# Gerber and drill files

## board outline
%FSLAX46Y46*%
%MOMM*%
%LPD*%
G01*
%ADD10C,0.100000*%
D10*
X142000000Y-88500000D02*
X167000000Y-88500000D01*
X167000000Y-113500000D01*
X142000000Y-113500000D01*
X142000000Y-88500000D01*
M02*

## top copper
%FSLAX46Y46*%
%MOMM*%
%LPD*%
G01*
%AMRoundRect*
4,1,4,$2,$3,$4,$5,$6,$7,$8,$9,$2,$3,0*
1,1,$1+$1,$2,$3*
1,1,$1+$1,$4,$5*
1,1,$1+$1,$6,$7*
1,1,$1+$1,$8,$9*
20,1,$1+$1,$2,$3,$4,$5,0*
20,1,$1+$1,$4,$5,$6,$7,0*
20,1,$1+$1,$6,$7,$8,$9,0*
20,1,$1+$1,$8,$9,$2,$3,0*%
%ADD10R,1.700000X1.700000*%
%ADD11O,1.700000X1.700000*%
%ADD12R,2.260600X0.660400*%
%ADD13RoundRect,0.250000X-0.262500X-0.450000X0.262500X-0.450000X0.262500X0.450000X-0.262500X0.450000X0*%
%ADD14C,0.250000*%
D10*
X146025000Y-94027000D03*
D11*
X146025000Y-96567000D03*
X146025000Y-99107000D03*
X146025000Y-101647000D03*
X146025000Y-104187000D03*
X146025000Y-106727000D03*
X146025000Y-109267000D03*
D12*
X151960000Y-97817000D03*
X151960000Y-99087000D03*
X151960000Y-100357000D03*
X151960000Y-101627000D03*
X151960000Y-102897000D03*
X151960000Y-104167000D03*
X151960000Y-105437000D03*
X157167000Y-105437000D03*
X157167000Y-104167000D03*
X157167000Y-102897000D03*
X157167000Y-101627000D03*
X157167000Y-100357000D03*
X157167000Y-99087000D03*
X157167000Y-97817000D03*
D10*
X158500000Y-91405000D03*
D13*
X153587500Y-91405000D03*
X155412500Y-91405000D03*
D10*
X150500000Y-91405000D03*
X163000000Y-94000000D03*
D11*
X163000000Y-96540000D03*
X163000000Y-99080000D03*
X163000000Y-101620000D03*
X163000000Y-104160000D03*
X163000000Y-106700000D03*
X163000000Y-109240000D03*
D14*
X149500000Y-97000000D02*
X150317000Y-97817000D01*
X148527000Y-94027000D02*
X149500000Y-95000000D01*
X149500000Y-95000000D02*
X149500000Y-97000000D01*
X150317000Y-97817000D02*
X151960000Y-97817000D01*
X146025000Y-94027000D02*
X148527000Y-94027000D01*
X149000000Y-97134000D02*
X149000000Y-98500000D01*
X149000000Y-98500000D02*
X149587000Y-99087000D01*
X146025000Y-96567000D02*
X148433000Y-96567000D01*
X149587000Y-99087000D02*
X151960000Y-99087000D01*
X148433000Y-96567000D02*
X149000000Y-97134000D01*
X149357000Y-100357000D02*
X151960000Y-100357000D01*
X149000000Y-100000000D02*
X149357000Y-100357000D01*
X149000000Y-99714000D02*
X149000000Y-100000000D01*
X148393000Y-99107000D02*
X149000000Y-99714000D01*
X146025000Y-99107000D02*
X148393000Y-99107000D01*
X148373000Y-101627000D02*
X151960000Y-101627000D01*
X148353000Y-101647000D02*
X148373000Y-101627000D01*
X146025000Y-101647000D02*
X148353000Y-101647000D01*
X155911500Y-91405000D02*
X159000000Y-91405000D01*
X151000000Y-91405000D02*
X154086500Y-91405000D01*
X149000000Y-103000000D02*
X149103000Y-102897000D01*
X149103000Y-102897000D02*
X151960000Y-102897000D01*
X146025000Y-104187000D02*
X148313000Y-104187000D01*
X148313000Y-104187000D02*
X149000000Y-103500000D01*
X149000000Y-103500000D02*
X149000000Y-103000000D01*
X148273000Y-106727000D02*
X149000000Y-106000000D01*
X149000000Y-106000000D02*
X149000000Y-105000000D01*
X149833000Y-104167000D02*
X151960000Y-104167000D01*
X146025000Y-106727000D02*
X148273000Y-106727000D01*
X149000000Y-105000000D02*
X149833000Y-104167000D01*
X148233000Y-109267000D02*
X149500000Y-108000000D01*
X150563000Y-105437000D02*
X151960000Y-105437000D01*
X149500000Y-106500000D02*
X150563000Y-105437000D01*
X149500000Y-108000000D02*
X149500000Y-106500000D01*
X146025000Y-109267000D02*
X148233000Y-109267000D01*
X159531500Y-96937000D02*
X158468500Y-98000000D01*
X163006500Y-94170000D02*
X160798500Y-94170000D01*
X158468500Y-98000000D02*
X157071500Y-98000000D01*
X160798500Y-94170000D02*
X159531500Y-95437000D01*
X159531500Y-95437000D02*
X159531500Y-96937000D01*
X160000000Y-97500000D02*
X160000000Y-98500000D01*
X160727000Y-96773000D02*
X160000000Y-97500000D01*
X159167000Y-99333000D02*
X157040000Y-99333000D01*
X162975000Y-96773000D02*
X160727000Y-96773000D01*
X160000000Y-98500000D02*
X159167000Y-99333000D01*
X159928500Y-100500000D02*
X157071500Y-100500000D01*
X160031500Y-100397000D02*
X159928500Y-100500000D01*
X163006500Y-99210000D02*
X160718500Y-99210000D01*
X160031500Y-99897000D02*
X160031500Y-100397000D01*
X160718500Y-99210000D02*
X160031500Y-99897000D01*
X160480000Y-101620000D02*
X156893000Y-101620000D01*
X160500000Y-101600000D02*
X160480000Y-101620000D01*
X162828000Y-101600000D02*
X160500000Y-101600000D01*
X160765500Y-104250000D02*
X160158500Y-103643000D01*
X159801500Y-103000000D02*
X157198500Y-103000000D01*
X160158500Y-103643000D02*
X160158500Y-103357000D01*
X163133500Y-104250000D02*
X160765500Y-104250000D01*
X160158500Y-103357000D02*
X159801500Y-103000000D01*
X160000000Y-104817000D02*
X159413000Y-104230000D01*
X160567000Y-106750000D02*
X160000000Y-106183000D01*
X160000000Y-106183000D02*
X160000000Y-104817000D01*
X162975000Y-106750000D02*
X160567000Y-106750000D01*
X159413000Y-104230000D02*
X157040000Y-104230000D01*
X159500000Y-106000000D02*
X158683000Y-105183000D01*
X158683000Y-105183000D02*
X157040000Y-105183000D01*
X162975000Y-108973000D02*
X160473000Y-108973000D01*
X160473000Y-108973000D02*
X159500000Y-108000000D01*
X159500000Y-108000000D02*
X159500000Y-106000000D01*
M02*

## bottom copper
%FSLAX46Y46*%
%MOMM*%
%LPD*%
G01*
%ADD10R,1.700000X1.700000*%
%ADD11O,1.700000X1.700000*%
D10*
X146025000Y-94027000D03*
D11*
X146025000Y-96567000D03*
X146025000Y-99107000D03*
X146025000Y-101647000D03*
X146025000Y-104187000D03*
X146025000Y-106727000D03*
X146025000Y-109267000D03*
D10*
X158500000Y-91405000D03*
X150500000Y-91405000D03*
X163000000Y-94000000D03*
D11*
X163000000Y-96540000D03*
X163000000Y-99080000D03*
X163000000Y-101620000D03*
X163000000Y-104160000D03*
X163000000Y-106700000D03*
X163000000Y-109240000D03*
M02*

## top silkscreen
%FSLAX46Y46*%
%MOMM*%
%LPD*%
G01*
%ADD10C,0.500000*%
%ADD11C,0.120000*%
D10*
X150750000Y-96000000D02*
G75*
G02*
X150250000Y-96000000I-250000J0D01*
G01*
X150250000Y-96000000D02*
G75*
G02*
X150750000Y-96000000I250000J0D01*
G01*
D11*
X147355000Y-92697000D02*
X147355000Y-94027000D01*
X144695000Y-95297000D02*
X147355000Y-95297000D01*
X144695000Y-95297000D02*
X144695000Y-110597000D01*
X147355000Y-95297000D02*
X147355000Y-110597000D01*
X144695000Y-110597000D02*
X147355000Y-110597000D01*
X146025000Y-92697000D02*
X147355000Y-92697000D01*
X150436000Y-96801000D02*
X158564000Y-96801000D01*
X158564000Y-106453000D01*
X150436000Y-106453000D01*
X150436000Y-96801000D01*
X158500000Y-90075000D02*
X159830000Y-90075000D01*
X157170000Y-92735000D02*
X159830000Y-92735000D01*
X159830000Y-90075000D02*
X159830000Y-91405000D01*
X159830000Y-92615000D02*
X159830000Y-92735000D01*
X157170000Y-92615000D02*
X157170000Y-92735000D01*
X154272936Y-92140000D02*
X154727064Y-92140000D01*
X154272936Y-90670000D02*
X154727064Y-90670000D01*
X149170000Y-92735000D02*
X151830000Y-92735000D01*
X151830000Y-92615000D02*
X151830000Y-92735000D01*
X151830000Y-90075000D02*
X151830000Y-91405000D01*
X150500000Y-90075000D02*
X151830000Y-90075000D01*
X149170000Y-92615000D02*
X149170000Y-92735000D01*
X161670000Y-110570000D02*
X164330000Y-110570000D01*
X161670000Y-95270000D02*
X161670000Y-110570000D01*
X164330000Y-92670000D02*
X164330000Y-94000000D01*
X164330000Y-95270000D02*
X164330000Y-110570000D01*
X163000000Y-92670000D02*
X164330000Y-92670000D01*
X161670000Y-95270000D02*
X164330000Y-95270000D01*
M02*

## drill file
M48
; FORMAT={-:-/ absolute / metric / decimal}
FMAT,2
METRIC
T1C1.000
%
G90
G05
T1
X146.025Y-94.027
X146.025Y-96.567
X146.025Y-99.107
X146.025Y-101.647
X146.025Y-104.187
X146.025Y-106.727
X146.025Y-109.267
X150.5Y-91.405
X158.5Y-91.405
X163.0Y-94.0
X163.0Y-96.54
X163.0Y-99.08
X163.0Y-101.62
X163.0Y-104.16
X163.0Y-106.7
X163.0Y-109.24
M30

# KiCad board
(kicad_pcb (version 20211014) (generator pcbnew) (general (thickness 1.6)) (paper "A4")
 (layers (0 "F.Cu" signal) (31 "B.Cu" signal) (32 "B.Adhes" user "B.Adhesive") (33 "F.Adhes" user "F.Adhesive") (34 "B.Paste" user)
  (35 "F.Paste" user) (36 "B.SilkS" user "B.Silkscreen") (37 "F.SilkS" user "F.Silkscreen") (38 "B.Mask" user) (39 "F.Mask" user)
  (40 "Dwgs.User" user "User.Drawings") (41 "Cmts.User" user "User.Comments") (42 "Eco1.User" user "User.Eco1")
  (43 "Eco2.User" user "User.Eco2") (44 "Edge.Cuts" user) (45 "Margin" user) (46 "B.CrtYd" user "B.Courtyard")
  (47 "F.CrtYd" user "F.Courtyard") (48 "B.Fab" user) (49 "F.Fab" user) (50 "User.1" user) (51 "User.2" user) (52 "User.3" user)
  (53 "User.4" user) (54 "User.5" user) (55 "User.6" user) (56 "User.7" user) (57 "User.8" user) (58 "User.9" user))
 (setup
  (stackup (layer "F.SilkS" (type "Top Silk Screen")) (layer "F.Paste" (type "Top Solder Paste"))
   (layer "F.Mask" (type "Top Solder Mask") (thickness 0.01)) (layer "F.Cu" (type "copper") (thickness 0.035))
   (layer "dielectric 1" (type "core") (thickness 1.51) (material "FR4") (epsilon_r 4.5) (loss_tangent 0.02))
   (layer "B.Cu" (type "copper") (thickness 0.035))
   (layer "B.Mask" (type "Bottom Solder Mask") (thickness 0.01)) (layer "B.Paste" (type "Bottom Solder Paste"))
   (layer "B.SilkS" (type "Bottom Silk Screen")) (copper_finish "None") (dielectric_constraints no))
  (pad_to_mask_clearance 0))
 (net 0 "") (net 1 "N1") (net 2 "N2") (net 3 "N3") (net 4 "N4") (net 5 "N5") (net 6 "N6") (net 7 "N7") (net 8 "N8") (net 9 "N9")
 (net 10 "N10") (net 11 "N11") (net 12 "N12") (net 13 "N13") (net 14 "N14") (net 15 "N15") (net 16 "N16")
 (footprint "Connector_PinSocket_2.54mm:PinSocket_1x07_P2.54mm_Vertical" (layer "F.Cu") (at 146.025 94.027)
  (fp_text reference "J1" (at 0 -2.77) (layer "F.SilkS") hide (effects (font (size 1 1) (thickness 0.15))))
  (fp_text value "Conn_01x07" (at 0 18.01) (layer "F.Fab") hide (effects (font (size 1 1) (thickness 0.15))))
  (fp_line (start 1.33 -1.33) (end 1.33 0) (layer "F.SilkS") (width 0.12))
  (fp_line (start -1.33 1.27) (end 1.33 1.27) (layer "F.SilkS") (width 0.12))
  (fp_line (start -1.33 1.27) (end -1.33 16.57) (layer "F.SilkS") (width 0.12))
  (fp_line (start 1.33 1.27) (end 1.33 16.57) (layer "F.SilkS") (width 0.12))
  (fp_line (start -1.33 16.57) (end 1.33 16.57) (layer "F.SilkS") (width 0.12))
  (fp_line (start 0 -1.33) (end 1.33 -1.33) (layer "F.SilkS") (width 0.12))
  (pad "1" thru_hole rect (at 0 0) (size 1.7 1.7) (drill 1) (layers *.Cu *.Mask) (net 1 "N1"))
  (pad "2" thru_hole oval (at 0 2.54) (size 1.7 1.7) (drill 1) (layers *.Cu *.Mask) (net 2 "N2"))
  (pad "3" thru_hole oval (at 0 5.08) (size 1.7 1.7) (drill 1) (layers *.Cu *.Mask) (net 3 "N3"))
  (pad "4" thru_hole oval (at 0 7.62) (size 1.7 1.7) (drill 1) (layers *.Cu *.Mask) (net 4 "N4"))
  (pad "5" thru_hole oval (at 0 10.16) (size 1.7 1.7) (drill 1) (layers *.Cu *.Mask) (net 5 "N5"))
  (pad "6" thru_hole oval (at 0 12.7) (size 1.7 1.7) (drill 1) (layers *.Cu *.Mask) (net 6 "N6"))
  (pad "7" thru_hole oval (at 0 15.24) (size 1.7 1.7) (drill 1) (layers *.Cu *.Mask) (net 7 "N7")))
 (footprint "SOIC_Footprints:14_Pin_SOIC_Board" (layer "F.Cu") (at 154.627 101.5)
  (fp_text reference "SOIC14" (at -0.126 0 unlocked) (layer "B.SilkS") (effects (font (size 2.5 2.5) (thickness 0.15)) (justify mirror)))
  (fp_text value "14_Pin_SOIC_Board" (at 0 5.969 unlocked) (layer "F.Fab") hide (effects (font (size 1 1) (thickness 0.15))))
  (fp_rect (start -4.191 -4.699) (end 3.937 4.953) (layer "F.SilkS") (width 0.12) (fill none))
  (pad "1" smd rect (at -2.667 -3.683) (size 2.2606 0.6604) (layers "F.Cu" "F.Paste" "F.Mask") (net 1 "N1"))
  (pad "2" smd rect (at -2.667 -2.413) (size 2.2606 0.6604) (layers "F.Cu" "F.Paste" "F.Mask") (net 2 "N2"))
  (pad "3" smd rect (at -2.667 -1.143) (size 2.2606 0.6604) (layers "F.Cu" "F.Paste" "F.Mask") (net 3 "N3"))
  (pad "4" smd rect (at -2.667 0.127) (size 2.2606 0.6604) (layers "F.Cu" "F.Paste" "F.Mask") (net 4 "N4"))
  (pad "5" smd rect (at -2.667 1.397) (size 2.2606 0.6604) (layers "F.Cu" "F.Paste" "F.Mask") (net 5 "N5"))
  (pad "6" smd rect (at -2.667 2.667) (size 2.2606 0.6604) (layers "F.Cu" "F.Paste" "F.Mask") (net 6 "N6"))
  (pad "7" smd rect (at -2.667 3.937) (size 2.2606 0.6604) (layers "F.Cu" "F.Paste" "F.Mask") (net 7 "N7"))
  (pad "8" smd rect (at 2.54 3.937) (size 2.2606 0.6604) (layers "F.Cu" "F.Paste" "F.Mask") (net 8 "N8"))
  (pad "9" smd rect (at 2.54 2.667) (size 2.2606 0.6604) (layers "F.Cu" "F.Paste" "F.Mask") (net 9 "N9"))
  (pad "10" smd rect (at 2.54 1.397) (size 2.2606 0.6604) (layers "F.Cu" "F.Paste" "F.Mask") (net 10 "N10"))
  (pad "11" smd rect (at 2.54 0.127) (size 2.2606 0.6604) (layers "F.Cu" "F.Paste" "F.Mask") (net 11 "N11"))
  (pad "12" smd rect (at 2.54 -1.143) (size 2.2606 0.6604) (layers "F.Cu" "F.Paste" "F.Mask") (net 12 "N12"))
  (pad "13" smd rect (at 2.54 -2.413) (size 2.2606 0.6604) (layers "F.Cu" "F.Paste" "F.Mask") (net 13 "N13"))
  (pad "14" smd rect (at 2.54 -3.683) (size 2.2606 0.6604) (layers "F.Cu" "F.Paste" "F.Mask") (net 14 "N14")))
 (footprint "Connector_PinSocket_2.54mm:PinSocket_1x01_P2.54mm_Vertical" (layer "F.Cu") (at 158.5 91.405)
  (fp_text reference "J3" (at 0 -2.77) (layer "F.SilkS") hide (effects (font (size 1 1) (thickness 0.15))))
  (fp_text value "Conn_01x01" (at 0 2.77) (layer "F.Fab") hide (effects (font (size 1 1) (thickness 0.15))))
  (fp_line (start 0 -1.33) (end 1.33 -1.33) (layer "F.SilkS") (width 0.12))
  (fp_line (start -1.33 1.33) (end 1.33 1.33) (layer "F.SilkS") (width 0.12))
  (fp_line (start 1.33 -1.33) (end 1.33 0) (layer "F.SilkS") (width 0.12))
  (fp_line (start 1.33 1.21) (end 1.33 1.33) (layer "F.SilkS") (width 0.12))
  (fp_line (start -1.33 1.21) (end -1.33 1.33) (layer "F.SilkS") (width 0.12))
  (pad "1" thru_hole rect (at 0 0) (size 1.7 1.7) (drill 1) (layers *.Cu *.Mask) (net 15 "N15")))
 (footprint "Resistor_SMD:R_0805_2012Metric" (layer "F.Cu") (at 154.5 91.405)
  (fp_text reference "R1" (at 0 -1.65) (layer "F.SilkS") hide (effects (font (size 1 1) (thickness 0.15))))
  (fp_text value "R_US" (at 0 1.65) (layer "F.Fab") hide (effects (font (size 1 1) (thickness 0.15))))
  (fp_line (start -0.227064 0.735) (end 0.227064 0.735) (layer "F.SilkS") (width 0.12))
  (fp_line (start -0.227064 -0.735) (end 0.227064 -0.735) (layer "F.SilkS") (width 0.12))
  (pad "1" smd roundrect (at -0.9125 0) (size 1.025 1.4) (layers "F.Cu" "F.Paste" "F.Mask") (roundrect_rratio 0.243902) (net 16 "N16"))
  (pad "2" smd roundrect (at 0.9125 0) (size 1.025 1.4) (layers "F.Cu" "F.Paste" "F.Mask") (roundrect_rratio 0.243902) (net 15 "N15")))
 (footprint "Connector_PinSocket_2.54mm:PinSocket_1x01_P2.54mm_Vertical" (layer "F.Cu") (at 150.5 91.405)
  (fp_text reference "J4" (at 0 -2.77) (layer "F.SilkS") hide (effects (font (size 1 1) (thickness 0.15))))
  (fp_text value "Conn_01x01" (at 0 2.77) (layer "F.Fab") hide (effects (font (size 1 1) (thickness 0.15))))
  (fp_line (start -1.33 1.33) (end 1.33 1.33) (layer "F.SilkS") (width 0.12))
  (fp_line (start 1.33 1.21) (end 1.33 1.33) (layer "F.SilkS") (width 0.12))
  (fp_line (start 1.33 -1.33) (end 1.33 0) (layer "F.SilkS") (width 0.12))
  (fp_line (start 0 -1.33) (end 1.33 -1.33) (layer "F.SilkS") (width 0.12))
  (fp_line (start -1.33 1.21) (end -1.33 1.33) (layer "F.SilkS") (width 0.12))
  (pad "1" thru_hole rect (at 0 0) (size 1.7 1.7) (drill 1) (layers *.Cu *.Mask) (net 16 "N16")))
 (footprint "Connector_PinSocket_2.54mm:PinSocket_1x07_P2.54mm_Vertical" (layer "F.Cu") (at 163 94)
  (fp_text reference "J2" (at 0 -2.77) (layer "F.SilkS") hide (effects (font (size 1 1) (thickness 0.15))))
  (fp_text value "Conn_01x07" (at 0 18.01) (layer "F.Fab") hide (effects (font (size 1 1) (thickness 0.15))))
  (fp_line (start -1.33 16.57) (end 1.33 16.57) (layer "F.SilkS") (width 0.12))
  (fp_line (start -1.33 1.27) (end -1.33 16.57) (layer "F.SilkS") (width 0.12))
  (fp_line (start 1.33 -1.33) (end 1.33 0) (layer "F.SilkS") (width 0.12))
  (fp_line (start 1.33 1.27) (end 1.33 16.57) (layer "F.SilkS") (width 0.12))
  (fp_line (start 0 -1.33) (end 1.33 -1.33) (layer "F.SilkS") (width 0.12))
  (fp_line (start -1.33 1.27) (end 1.33 1.27) (layer "F.SilkS") (width 0.12))
  (pad "1" thru_hole rect (at 0 0) (size 1.7 1.7) (drill 1) (layers *.Cu *.Mask) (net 14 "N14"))
  (pad "2" thru_hole oval (at 0 2.54) (size 1.7 1.7) (drill 1) (layers *.Cu *.Mask) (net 13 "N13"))
  (pad "3" thru_hole oval (at 0 5.08) (size 1.7 1.7) (drill 1) (layers *.Cu *.Mask) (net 12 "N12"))
  (pad "4" thru_hole oval (at 0 7.62) (size 1.7 1.7) (drill 1) (layers *.Cu *.Mask) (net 11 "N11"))
  (pad "5" thru_hole oval (at 0 10.16) (size 1.7 1.7) (drill 1) (layers *.Cu *.Mask) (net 10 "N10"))
  (pad "6" thru_hole oval (at 0 12.7) (size 1.7 1.7) (drill 1) (layers *.Cu *.Mask) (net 9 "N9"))
  (pad "7" thru_hole oval (at 0 15.24) (size 1.7 1.7) (drill 1) (layers *.Cu *.Mask) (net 8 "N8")))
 (gr_circle (center 150.5 96) (end 150.9 96) (layer "F.SilkS") (width 0.2) (fill solid))
 (gr_rect (start 142 88.5) (end 167 113.5) (layer "Edge.Cuts") (width 0.1) (fill none))
 (segment (start 149.5 97) (end 150.317 97.817) (width 0.25) (layer "F.Cu") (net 1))
 (segment (start 148.527 94.027) (end 149.5 95) (width 0.25) (layer "F.Cu") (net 1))
 (segment (start 149.5 95) (end 149.5 97) (width 0.25) (layer "F.Cu") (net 1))
 (segment (start 150.317 97.817) (end 151.96 97.817) (width 0.25) (layer "F.Cu") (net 1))
 (segment (start 146.025 94.027) (end 148.527 94.027) (width 0.25) (layer "F.Cu") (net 1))
 (segment (start 149 97.134) (end 149 98.5) (width 0.25) (layer "F.Cu") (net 2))
 (segment (start 149 98.5) (end 149.587 99.087) (width 0.25) (layer "F.Cu") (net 2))
 (segment (start 146.025 96.567) (end 148.433 96.567) (width 0.25) (layer "F.Cu") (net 2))
 (segment (start 149.587 99.087) (end 151.96 99.087) (width 0.25) (layer "F.Cu") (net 2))
 (segment (start 148.433 96.567) (end 149 97.134) (width 0.25) (layer "F.Cu") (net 2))
 (segment (start 149.357 100.357) (end 151.96 100.357) (width 0.25) (layer "F.Cu") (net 3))
 (segment (start 149 100) (end 149.357 100.357) (width 0.25) (layer "F.Cu") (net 3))
 (segment (start 149 99.714) (end 149 100) (width 0.25) (layer "F.Cu") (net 3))
 (segment (start 148.393 99.107) (end 149 99.714) (width 0.25) (layer "F.Cu") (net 3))
 (segment (start 146.025 99.107) (end 148.393 99.107) (width 0.25) (layer "F.Cu") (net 3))
 (segment (start 148.373 101.627) (end 151.96 101.627) (width 0.25) (layer "F.Cu") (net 4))
 (segment (start 148.353 101.647) (end 148.373 101.627) (width 0.25) (layer "F.Cu") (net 4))
 (segment (start 146.025 101.647) (end 148.353 101.647) (width 0.25) (layer "F.Cu") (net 4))
 (segment (start 155.9115 91.405) (end 159 91.405) (width 0.25) (layer "F.Cu") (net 15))
 (segment (start 151 91.405) (end 154.0865 91.405) (width 0.25) (layer "F.Cu") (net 16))
 (segment (start 149 103) (end 149.103 102.897) (width 0.25) (layer "F.Cu") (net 5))
 (segment (start 149.103 102.897) (end 151.96 102.897) (width 0.25) (layer "F.Cu") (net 5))
 (segment (start 146.025 104.187) (end 148.313 104.187) (width 0.25) (layer "F.Cu") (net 5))
 (segment (start 148.313 104.187) (end 149 103.5) (width 0.25) (layer "F.Cu") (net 5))
 (segment (start 149 103.5) (end 149 103) (width 0.25) (layer "F.Cu") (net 5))
 (segment (start 148.273 106.727) (end 149 106) (width 0.25) (layer "F.Cu") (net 6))
 (segment (start 149 106) (end 149 105) (width 0.25) (layer "F.Cu") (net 6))
 (segment (start 149.833 104.167) (end 151.96 104.167) (width 0.25) (layer "F.Cu") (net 6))
 (segment (start 146.025 106.727) (end 148.273 106.727) (width 0.25) (layer "F.Cu") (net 6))
 (segment (start 149 105) (end 149.833 104.167) (width 0.25) (layer "F.Cu") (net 6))
 (segment (start 148.233 109.267) (end 149.5 108) (width 0.25) (layer "F.Cu") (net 7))
 (segment (start 150.563 105.437) (end 151.96 105.437) (width 0.25) (layer "F.Cu") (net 7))
 (segment (start 149.5 106.5) (end 150.563 105.437) (width 0.25) (layer "F.Cu") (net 7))
 (segment (start 149.5 108) (end 149.5 106.5) (width 0.25) (layer "F.Cu") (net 7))
 (segment (start 146.025 109.267) (end 148.233 109.267) (width 0.25) (layer "F.Cu") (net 7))
 (segment (start 159.5315 96.937) (end 158.4685 98) (width 0.25) (layer "F.Cu") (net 14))
 (segment (start 163.0065 94.17) (end 160.7985 94.17) (width 0.25) (layer "F.Cu") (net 14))
 (segment (start 158.4685 98) (end 157.0715 98) (width 0.25) (layer "F.Cu") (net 14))
 (segment (start 160.7985 94.17) (end 159.5315 95.437) (width 0.25) (layer "F.Cu") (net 14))
 (segment (start 159.5315 95.437) (end 159.5315 96.937) (width 0.25) (layer "F.Cu") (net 14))
 (segment (start 160 97.5) (end 160 98.5) (width 0.25) (layer "F.Cu") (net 13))
 (segment (start 160.727 96.773) (end 160 97.5) (width 0.25) (layer "F.Cu") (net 13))
 (segment (start 159.167 99.333) (end 157.04 99.333) (width 0.25) (layer "F.Cu") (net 13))
 (segment (start 162.975 96.773) (end 160.727 96.773) (width 0.25) (layer "F.Cu") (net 13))
 (segment (start 160 98.5) (end 159.167 99.333) (width 0.25) (layer "F.Cu") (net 13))
 (segment (start 159.9285 100.5) (end 157.0715 100.5) (width 0.25) (layer "F.Cu") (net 12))
 (segment (start 160.0315 100.397) (end 159.9285 100.5) (width 0.25) (layer "F.Cu") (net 12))
 (segment (start 163.0065 99.21) (end 160.7185 99.21) (width 0.25) (layer "F.Cu") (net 12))
 (segment (start 160.0315 99.897) (end 160.0315 100.397) (width 0.25) (layer "F.Cu") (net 12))
 (segment (start 160.7185 99.21) (end 160.0315 99.897) (width 0.25) (layer "F.Cu") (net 12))
 (segment (start 160.48 101.62) (end 156.893 101.62) (width 0.25) (layer "F.Cu") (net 11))
 (segment (start 160.5 101.6) (end 160.48 101.62) (width 0.25) (layer "F.Cu") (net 11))
 (segment (start 162.828 101.6) (end 160.5 101.6) (width 0.25) (layer "F.Cu") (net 11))
 (segment (start 160.7655 104.25) (end 160.1585 103.643) (width 0.25) (layer "F.Cu") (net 10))
 (segment (start 159.8015 103) (end 157.1985 103) (width 0.25) (layer "F.Cu") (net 10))
 (segment (start 160.1585 103.643) (end 160.1585 103.357) (width 0.25) (layer "F.Cu") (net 10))
 (segment (start 163.1335 104.25) (end 160.7655 104.25) (width 0.25) (layer "F.Cu") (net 10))
 (segment (start 160.1585 103.357) (end 159.8015 103) (width 0.25) (layer "F.Cu") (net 10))
 (segment (start 160 104.817) (end 159.413 104.23) (width 0.25) (layer "F.Cu") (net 9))
 (segment (start 160.567 106.75) (end 160 106.183) (width 0.25) (layer "F.Cu") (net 9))
 (segment (start 160 106.183) (end 160 104.817) (width 0.25) (layer "F.Cu") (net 9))
 (segment (start 162.975 106.75) (end 160.567 106.75) (width 0.25) (layer "F.Cu") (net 9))
 (segment (start 159.413 104.23) (end 157.04 104.23) (width 0.25) (layer "F.Cu") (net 9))
 (segment (start 159.5 106) (end 158.683 105.183) (width 0.25) (layer "F.Cu") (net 8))
 (segment (start 158.683 105.183) (end 157.04 105.183) (width 0.25) (layer "F.Cu") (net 8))
 (segment (start 162.975 108.973) (end 160.473 108.973) (width 0.25) (layer "F.Cu") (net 8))
 (segment (start 160.473 108.973) (end 159.5 108) (width 0.25) (layer "F.Cu") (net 8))
 (segment (start 159.5 108) (end 159.5 106) (width 0.25) (layer "F.Cu") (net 8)))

